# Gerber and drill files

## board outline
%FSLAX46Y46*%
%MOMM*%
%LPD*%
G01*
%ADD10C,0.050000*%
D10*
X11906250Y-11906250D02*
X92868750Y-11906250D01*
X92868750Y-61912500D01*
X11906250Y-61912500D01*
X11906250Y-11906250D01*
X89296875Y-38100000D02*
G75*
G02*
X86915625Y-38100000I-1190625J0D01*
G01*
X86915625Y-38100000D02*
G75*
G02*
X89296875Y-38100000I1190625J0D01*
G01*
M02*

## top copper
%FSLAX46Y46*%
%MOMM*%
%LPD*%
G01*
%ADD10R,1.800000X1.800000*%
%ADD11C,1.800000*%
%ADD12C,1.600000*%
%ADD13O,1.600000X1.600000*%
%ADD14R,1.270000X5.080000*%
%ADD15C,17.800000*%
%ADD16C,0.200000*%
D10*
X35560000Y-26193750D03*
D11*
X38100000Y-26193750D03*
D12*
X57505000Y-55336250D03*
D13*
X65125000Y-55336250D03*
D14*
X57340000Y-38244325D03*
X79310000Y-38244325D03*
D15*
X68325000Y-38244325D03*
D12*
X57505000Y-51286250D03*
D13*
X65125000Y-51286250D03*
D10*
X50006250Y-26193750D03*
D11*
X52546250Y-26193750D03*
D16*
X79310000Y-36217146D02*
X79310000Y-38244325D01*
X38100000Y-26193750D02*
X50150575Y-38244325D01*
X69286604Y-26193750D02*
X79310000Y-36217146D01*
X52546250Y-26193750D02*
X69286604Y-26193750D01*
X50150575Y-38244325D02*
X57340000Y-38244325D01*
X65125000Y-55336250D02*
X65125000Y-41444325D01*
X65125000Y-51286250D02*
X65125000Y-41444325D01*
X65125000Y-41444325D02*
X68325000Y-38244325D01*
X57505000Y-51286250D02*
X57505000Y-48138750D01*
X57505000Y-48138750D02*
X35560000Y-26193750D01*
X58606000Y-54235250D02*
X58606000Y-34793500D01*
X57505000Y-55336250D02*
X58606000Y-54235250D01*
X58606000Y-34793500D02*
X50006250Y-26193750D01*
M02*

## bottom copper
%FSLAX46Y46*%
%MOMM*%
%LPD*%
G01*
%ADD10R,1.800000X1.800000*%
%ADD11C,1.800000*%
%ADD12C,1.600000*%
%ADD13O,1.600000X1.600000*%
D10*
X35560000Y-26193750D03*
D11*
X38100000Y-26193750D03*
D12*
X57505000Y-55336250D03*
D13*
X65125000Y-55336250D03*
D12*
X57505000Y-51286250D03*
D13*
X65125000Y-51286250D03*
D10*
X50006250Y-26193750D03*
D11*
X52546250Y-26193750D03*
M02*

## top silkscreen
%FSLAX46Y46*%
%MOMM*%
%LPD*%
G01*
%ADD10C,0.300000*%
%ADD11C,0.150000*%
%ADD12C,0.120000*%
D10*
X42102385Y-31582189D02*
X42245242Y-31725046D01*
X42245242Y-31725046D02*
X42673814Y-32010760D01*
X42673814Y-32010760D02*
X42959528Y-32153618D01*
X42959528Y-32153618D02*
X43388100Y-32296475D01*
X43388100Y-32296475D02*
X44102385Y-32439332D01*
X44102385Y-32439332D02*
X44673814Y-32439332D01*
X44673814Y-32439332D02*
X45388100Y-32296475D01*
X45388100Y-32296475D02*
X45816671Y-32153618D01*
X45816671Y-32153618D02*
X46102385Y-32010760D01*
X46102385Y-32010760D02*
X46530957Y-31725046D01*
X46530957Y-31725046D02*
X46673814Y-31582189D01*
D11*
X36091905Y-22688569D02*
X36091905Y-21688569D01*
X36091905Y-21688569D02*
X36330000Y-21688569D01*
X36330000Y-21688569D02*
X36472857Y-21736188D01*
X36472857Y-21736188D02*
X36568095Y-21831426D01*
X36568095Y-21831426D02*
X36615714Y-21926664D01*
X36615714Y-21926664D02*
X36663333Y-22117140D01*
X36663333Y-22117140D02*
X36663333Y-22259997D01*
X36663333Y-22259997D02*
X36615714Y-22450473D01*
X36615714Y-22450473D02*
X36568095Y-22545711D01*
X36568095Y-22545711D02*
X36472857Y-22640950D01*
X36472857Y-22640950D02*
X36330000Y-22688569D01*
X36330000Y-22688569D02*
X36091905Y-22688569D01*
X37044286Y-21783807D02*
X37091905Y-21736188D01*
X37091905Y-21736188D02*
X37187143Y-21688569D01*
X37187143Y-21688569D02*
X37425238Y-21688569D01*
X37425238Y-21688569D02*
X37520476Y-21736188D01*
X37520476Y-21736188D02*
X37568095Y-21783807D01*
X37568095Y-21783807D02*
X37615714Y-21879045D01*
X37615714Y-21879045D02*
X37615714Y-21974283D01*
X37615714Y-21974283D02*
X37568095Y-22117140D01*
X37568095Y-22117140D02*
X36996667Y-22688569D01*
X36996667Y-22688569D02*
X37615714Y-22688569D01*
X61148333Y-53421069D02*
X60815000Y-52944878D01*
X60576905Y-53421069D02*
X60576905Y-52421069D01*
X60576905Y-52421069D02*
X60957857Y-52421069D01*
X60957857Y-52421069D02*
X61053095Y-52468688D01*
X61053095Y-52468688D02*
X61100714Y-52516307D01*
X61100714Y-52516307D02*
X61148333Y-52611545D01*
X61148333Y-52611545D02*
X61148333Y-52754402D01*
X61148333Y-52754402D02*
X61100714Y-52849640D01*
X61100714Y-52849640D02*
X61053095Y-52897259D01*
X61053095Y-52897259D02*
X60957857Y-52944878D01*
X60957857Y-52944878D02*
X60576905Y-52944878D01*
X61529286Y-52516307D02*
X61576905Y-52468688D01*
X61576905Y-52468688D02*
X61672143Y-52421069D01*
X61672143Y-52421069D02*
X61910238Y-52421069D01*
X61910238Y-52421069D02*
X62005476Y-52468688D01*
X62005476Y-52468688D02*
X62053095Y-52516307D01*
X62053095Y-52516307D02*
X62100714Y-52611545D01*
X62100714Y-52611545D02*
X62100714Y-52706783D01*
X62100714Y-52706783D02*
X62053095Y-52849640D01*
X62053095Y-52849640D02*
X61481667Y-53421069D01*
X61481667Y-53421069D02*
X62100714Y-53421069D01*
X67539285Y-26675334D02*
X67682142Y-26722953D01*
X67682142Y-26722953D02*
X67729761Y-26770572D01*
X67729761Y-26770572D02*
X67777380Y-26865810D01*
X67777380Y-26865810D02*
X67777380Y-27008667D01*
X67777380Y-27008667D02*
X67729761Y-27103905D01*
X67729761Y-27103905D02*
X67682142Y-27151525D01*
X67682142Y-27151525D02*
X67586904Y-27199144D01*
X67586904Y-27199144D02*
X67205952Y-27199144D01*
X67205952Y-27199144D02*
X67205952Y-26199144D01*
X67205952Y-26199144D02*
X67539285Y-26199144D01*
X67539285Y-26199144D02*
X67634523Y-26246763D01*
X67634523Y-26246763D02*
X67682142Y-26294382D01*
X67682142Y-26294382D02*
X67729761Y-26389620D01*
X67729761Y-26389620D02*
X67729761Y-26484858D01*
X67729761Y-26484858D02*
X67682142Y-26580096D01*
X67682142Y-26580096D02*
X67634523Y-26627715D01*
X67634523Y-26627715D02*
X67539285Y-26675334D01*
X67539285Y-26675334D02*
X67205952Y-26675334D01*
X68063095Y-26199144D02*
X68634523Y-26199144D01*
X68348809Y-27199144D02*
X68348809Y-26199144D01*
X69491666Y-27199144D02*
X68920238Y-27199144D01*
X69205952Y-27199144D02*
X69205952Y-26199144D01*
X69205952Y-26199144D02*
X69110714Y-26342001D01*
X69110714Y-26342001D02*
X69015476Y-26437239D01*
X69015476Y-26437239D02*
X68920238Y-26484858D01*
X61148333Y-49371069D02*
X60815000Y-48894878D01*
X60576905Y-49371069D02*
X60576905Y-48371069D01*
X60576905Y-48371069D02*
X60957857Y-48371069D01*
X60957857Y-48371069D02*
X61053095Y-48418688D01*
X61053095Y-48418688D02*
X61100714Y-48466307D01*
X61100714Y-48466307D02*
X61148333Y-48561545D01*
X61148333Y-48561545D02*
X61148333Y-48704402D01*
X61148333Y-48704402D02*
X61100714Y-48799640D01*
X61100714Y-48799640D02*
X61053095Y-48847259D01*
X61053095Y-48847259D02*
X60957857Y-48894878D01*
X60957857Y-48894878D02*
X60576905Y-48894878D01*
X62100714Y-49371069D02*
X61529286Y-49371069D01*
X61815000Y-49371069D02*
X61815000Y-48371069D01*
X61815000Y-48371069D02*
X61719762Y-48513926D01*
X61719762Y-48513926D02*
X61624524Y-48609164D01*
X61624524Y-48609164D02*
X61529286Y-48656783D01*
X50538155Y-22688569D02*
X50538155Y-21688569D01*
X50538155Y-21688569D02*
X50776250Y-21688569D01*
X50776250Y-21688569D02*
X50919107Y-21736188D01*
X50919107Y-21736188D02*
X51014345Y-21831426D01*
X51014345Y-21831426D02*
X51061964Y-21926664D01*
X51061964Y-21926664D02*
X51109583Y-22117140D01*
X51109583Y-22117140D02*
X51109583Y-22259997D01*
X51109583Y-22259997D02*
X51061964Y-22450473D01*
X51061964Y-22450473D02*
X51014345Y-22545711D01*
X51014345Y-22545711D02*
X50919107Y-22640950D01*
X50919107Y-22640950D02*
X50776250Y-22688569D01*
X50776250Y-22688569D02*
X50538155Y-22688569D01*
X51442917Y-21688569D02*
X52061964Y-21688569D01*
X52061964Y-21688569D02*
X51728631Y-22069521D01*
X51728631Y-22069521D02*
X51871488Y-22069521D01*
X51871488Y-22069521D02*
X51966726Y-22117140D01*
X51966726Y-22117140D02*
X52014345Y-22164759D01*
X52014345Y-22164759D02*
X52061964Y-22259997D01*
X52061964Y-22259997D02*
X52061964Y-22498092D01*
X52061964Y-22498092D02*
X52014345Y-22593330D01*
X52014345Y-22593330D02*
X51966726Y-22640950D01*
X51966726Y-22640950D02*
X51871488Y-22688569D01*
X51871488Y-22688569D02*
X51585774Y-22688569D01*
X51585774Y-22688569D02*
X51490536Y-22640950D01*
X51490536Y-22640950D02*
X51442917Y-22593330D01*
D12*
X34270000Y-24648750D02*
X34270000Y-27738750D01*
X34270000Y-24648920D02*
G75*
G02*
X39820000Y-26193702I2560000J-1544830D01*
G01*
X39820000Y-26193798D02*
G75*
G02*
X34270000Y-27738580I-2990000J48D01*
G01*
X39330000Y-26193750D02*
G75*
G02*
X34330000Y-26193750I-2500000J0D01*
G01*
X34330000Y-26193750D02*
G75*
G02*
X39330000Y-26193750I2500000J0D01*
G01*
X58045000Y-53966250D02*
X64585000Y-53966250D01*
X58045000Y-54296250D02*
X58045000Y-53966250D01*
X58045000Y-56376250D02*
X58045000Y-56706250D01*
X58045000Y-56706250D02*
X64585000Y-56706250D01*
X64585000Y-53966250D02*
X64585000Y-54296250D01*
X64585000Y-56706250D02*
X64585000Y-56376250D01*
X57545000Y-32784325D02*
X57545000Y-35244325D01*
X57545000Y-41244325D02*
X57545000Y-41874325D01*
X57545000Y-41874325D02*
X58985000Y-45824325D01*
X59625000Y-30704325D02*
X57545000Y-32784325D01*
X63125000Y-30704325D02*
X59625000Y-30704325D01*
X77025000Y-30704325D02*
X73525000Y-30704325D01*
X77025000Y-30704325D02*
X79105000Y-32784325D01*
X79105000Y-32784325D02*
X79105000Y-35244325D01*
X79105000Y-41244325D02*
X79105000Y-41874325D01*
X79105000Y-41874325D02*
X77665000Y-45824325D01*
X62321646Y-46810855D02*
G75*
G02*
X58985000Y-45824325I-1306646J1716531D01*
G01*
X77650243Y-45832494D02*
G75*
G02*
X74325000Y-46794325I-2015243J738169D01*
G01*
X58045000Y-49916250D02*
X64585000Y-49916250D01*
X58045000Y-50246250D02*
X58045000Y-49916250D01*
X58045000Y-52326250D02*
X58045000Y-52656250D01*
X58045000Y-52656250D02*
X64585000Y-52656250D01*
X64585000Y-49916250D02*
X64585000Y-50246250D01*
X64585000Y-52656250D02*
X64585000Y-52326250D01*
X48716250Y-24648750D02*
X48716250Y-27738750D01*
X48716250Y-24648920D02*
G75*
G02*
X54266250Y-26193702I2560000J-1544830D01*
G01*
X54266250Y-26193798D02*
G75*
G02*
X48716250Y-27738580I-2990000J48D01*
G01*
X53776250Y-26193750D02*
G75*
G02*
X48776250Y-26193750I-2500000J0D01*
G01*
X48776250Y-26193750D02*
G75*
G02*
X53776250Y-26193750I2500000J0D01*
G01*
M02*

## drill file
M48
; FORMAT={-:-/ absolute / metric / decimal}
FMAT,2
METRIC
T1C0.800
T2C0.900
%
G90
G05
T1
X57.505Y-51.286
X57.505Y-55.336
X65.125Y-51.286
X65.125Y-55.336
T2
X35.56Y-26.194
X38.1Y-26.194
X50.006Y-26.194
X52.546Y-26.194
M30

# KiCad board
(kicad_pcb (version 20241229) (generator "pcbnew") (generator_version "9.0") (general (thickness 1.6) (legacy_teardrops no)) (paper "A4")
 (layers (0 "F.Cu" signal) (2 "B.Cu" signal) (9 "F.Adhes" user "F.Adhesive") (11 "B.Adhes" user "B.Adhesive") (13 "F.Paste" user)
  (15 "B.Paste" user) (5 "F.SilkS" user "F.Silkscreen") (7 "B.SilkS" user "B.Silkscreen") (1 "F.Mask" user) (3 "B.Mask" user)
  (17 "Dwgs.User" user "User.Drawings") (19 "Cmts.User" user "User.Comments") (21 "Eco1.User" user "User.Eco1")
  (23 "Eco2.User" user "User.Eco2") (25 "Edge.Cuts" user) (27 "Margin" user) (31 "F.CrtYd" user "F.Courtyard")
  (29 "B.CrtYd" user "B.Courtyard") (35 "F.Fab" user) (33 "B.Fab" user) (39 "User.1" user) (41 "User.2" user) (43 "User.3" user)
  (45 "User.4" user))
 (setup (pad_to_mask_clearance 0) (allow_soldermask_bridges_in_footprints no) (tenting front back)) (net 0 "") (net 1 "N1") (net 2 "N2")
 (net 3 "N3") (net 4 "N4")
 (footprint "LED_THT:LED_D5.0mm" (layer "F.Cu") (at 35.56 26.19375)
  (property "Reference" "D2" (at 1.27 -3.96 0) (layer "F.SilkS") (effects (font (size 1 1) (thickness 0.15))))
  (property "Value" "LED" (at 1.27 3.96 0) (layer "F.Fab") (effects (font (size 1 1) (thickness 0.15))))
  (fp_line (start -1.29 -1.545) (end -1.29 1.545) (stroke (width 0.12) (type solid)) (layer "F.SilkS"))
  (fp_arc (start -1.29 -1.54483) (mid 2.071756 -2.880501) (end 4.26 -0.000048) (stroke (width 0.12) (type solid)) (layer "F.SilkS"))
  (fp_arc (start 4.26 0.000048) (mid 2.071756 2.880501) (end -1.29 1.54483) (stroke (width 0.12) (type solid)) (layer "F.SilkS"))
  (fp_circle (center 1.27 0) (end 3.77 0) (stroke (width 0.12) (type solid)) (fill no) (layer "F.SilkS"))
  (pad "1" thru_hole rect (at 0 0) (size 1.8 1.8) (drill 0.9) (layers "*.Cu" "*.Mask") (remove_unused_layers no) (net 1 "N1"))
  (pad "2" thru_hole circle (at 2.54 0) (size 1.8 1.8) (drill 0.9) (layers "*.Cu" "*.Mask") (remove_unused_layers no) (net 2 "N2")))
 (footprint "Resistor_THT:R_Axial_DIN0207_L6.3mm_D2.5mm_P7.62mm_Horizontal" (layer "F.Cu") (at 57.505 55.33625)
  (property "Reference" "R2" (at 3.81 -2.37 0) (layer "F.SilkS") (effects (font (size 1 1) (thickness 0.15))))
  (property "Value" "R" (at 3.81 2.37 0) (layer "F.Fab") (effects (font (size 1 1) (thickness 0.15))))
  (fp_line (start 0.54 -1.37) (end 7.08 -1.37) (stroke (width 0.12) (type solid)) (layer "F.SilkS"))
  (fp_line (start 0.54 -1.04) (end 0.54 -1.37) (stroke (width 0.12) (type solid)) (layer "F.SilkS"))
  (fp_line (start 0.54 1.04) (end 0.54 1.37) (stroke (width 0.12) (type solid)) (layer "F.SilkS"))
  (fp_line (start 0.54 1.37) (end 7.08 1.37) (stroke (width 0.12) (type solid)) (layer "F.SilkS"))
  (fp_line (start 7.08 -1.37) (end 7.08 -1.04) (stroke (width 0.12) (type solid)) (layer "F.SilkS"))
  (fp_line (start 7.08 1.37) (end 7.08 1.04) (stroke (width 0.12) (type solid)) (layer "F.SilkS"))
  (pad "1" thru_hole circle (at 0 0) (size 1.6 1.6) (drill 0.8) (layers "*.Cu" "*.Mask") (remove_unused_layers no) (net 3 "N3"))
  (pad "2" thru_hole oval (at 7.62 0) (size 1.6 1.6) (drill 0.8) (layers "*.Cu" "*.Mask") (remove_unused_layers no) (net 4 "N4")))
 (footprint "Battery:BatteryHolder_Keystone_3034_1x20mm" (layer "F.Cu") (at 68.325 38.244325)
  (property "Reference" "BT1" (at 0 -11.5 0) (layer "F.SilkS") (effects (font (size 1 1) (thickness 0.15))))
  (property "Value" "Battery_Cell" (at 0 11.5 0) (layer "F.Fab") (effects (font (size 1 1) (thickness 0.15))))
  (fp_line (start -10.78 -5.46) (end -10.78 -3) (stroke (width 0.12) (type solid)) (layer "F.SilkS"))
  (fp_line (start -10.78 3) (end -10.78 3.63) (stroke (width 0.12) (type solid)) (layer "F.SilkS"))
  (fp_line (start -10.78 3.63) (end -9.34 7.58) (stroke (width 0.12) (type solid)) (layer "F.SilkS"))
  (fp_line (start -8.7 -7.54) (end -10.78 -5.46) (stroke (width 0.12) (type solid)) (layer "F.SilkS"))
  (fp_line (start -5.2 -7.54) (end -8.7 -7.54) (stroke (width 0.12) (type solid)) (layer "F.SilkS"))
  (fp_line (start 8.7 -7.54) (end 5.2 -7.54) (stroke (width 0.12) (type solid)) (layer "F.SilkS"))
  (fp_line (start 8.7 -7.54) (end 10.78 -5.46) (stroke (width 0.12) (type solid)) (layer "F.SilkS"))
  (fp_line (start 10.78 -5.46) (end 10.78 -3) (stroke (width 0.12) (type solid)) (layer "F.SilkS"))
  (fp_line (start 10.78 3) (end 10.78 3.63) (stroke (width 0.12) (type solid)) (layer "F.SilkS"))
  (fp_line (start 10.78 3.63) (end 9.34 7.58) (stroke (width 0.12) (type solid)) (layer "F.SilkS"))
  (fp_arc (start -6.003354 8.56653) (mid -7.921654 8.918738) (end -9.34 7.58) (stroke (width 0.12) (type solid)) (layer "F.SilkS"))
  (fp_arc (start 9.325243 7.588169) (mid 7.90634 8.911668) (end 6 8.55) (stroke (width 0.12) (type solid)) (layer "F.SilkS"))
  (pad "1" smd rect (at -10.985 0) (size 1.27 5.08) (layers "F.Cu" "F.Mask" "F.Paste") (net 2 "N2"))
  (pad "1" smd rect (at 10.985 0) (size 1.27 5.08) (layers "F.Cu" "F.Mask" "F.Paste") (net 2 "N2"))
  (pad "2" smd circle (at 0 0) (size 17.8 17.8) (layers "F.Cu" "F.Mask") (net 4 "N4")))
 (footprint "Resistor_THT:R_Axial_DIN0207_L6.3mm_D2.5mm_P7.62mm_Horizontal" (layer "F.Cu") (at 57.505 51.28625)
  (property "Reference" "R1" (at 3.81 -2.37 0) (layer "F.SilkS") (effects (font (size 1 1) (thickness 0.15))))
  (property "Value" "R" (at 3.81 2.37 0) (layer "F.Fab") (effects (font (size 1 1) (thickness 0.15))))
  (fp_line (start 0.54 -1.37) (end 7.08 -1.37) (stroke (width 0.12) (type solid)) (layer "F.SilkS"))
  (fp_line (start 0.54 -1.04) (end 0.54 -1.37) (stroke (width 0.12) (type solid)) (layer "F.SilkS"))
  (fp_line (start 0.54 1.04) (end 0.54 1.37) (stroke (width 0.12) (type solid)) (layer "F.SilkS"))
  (fp_line (start 0.54 1.37) (end 7.08 1.37) (stroke (width 0.12) (type solid)) (layer "F.SilkS"))
  (fp_line (start 7.08 -1.37) (end 7.08 -1.04) (stroke (width 0.12) (type solid)) (layer "F.SilkS"))
  (fp_line (start 7.08 1.37) (end 7.08 1.04) (stroke (width 0.12) (type solid)) (layer "F.SilkS"))
  (pad "1" thru_hole circle (at 0 0) (size 1.6 1.6) (drill 0.8) (layers "*.Cu" "*.Mask") (remove_unused_layers no) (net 1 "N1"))
  (pad "2" thru_hole oval (at 7.62 0) (size 1.6 1.6) (drill 0.8) (layers "*.Cu" "*.Mask") (remove_unused_layers no) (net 4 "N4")))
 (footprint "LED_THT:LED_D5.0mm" (layer "F.Cu") (at 50.00625 26.19375)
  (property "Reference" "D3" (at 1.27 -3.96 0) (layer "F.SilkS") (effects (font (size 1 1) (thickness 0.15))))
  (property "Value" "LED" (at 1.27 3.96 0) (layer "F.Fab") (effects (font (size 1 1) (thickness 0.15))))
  (fp_line (start -1.29 -1.545) (end -1.29 1.545) (stroke (width 0.12) (type solid)) (layer "F.SilkS"))
  (fp_arc (start -1.29 -1.54483) (mid 2.071756 -2.880501) (end 4.26 -0.000048) (stroke (width 0.12) (type solid)) (layer "F.SilkS"))
  (fp_arc (start 4.26 0.000048) (mid 2.071756 2.880501) (end -1.29 1.54483) (stroke (width 0.12) (type solid)) (layer "F.SilkS"))
  (fp_circle (center 1.27 0) (end 3.77 0) (stroke (width 0.12) (type solid)) (fill no) (layer "F.SilkS"))
  (pad "1" thru_hole rect (at 0 0) (size 1.8 1.8) (drill 0.9) (layers "*.Cu" "*.Mask") (remove_unused_layers no) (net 3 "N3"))
  (pad "2" thru_hole circle (at 2.54 0) (size 1.8 1.8) (drill 0.9) (layers "*.Cu" "*.Mask") (remove_unused_layers no) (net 2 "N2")))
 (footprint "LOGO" (layer "B.Cu") (at 21.43125 40.48125 180)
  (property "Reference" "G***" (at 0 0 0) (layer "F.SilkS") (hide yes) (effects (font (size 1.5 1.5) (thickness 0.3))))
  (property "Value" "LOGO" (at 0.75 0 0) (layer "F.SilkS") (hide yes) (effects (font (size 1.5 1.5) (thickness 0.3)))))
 (gr_rect (start 11.90625 11.90625) (end 92.86875 61.9125) (stroke (width 0.05) (type default)) (fill no) (layer "Edge.Cuts"))
 (gr_circle (center 88.10625 38.1) (end 88.10625 39.290625) (stroke (width 0.05) (type default)) (fill no) (layer "Edge.Cuts"))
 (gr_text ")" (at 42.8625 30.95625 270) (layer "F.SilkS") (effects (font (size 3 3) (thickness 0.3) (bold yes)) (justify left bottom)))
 (segment (start 79.31 36.217146) (end 79.31 38.244325) (width 0.2) (layer "F.Cu") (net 2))
 (segment (start 38.1 26.19375) (end 50.150575 38.244325) (width 0.2) (layer "F.Cu") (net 2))
 (segment (start 69.286604 26.19375) (end 79.31 36.217146) (width 0.2) (layer "F.Cu") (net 2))
 (segment (start 52.54625 26.19375) (end 69.286604 26.19375) (width 0.2) (layer "F.Cu") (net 2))
 (segment (start 50.150575 38.244325) (end 57.34 38.244325) (width 0.2) (layer "F.Cu") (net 2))
 (segment (start 65.125 55.33625) (end 65.125 41.444325) (width 0.2) (layer "F.Cu") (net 4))
 (segment (start 65.125 51.28625) (end 65.125 41.444325) (width 0.2) (layer "F.Cu") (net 4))
 (segment (start 65.125 41.444325) (end 68.325 38.244325) (width 0.2) (layer "F.Cu") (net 4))
 (segment (start 57.505 51.28625) (end 57.505 48.13875) (width 0.2) (layer "F.Cu") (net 1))
 (segment (start 57.505 48.13875) (end 35.56 26.19375) (width 0.2) (layer "F.Cu") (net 1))
 (segment (start 58.606 54.23525) (end 58.606 34.7935) (width 0.2) (layer "F.Cu") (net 3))
 (segment (start 57.505 55.33625) (end 58.606 54.23525) (width 0.2) (layer "F.Cu") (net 3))
 (segment (start 58.606 34.7935) (end 50.00625 26.19375) (width 0.2) (layer "F.Cu") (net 3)))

